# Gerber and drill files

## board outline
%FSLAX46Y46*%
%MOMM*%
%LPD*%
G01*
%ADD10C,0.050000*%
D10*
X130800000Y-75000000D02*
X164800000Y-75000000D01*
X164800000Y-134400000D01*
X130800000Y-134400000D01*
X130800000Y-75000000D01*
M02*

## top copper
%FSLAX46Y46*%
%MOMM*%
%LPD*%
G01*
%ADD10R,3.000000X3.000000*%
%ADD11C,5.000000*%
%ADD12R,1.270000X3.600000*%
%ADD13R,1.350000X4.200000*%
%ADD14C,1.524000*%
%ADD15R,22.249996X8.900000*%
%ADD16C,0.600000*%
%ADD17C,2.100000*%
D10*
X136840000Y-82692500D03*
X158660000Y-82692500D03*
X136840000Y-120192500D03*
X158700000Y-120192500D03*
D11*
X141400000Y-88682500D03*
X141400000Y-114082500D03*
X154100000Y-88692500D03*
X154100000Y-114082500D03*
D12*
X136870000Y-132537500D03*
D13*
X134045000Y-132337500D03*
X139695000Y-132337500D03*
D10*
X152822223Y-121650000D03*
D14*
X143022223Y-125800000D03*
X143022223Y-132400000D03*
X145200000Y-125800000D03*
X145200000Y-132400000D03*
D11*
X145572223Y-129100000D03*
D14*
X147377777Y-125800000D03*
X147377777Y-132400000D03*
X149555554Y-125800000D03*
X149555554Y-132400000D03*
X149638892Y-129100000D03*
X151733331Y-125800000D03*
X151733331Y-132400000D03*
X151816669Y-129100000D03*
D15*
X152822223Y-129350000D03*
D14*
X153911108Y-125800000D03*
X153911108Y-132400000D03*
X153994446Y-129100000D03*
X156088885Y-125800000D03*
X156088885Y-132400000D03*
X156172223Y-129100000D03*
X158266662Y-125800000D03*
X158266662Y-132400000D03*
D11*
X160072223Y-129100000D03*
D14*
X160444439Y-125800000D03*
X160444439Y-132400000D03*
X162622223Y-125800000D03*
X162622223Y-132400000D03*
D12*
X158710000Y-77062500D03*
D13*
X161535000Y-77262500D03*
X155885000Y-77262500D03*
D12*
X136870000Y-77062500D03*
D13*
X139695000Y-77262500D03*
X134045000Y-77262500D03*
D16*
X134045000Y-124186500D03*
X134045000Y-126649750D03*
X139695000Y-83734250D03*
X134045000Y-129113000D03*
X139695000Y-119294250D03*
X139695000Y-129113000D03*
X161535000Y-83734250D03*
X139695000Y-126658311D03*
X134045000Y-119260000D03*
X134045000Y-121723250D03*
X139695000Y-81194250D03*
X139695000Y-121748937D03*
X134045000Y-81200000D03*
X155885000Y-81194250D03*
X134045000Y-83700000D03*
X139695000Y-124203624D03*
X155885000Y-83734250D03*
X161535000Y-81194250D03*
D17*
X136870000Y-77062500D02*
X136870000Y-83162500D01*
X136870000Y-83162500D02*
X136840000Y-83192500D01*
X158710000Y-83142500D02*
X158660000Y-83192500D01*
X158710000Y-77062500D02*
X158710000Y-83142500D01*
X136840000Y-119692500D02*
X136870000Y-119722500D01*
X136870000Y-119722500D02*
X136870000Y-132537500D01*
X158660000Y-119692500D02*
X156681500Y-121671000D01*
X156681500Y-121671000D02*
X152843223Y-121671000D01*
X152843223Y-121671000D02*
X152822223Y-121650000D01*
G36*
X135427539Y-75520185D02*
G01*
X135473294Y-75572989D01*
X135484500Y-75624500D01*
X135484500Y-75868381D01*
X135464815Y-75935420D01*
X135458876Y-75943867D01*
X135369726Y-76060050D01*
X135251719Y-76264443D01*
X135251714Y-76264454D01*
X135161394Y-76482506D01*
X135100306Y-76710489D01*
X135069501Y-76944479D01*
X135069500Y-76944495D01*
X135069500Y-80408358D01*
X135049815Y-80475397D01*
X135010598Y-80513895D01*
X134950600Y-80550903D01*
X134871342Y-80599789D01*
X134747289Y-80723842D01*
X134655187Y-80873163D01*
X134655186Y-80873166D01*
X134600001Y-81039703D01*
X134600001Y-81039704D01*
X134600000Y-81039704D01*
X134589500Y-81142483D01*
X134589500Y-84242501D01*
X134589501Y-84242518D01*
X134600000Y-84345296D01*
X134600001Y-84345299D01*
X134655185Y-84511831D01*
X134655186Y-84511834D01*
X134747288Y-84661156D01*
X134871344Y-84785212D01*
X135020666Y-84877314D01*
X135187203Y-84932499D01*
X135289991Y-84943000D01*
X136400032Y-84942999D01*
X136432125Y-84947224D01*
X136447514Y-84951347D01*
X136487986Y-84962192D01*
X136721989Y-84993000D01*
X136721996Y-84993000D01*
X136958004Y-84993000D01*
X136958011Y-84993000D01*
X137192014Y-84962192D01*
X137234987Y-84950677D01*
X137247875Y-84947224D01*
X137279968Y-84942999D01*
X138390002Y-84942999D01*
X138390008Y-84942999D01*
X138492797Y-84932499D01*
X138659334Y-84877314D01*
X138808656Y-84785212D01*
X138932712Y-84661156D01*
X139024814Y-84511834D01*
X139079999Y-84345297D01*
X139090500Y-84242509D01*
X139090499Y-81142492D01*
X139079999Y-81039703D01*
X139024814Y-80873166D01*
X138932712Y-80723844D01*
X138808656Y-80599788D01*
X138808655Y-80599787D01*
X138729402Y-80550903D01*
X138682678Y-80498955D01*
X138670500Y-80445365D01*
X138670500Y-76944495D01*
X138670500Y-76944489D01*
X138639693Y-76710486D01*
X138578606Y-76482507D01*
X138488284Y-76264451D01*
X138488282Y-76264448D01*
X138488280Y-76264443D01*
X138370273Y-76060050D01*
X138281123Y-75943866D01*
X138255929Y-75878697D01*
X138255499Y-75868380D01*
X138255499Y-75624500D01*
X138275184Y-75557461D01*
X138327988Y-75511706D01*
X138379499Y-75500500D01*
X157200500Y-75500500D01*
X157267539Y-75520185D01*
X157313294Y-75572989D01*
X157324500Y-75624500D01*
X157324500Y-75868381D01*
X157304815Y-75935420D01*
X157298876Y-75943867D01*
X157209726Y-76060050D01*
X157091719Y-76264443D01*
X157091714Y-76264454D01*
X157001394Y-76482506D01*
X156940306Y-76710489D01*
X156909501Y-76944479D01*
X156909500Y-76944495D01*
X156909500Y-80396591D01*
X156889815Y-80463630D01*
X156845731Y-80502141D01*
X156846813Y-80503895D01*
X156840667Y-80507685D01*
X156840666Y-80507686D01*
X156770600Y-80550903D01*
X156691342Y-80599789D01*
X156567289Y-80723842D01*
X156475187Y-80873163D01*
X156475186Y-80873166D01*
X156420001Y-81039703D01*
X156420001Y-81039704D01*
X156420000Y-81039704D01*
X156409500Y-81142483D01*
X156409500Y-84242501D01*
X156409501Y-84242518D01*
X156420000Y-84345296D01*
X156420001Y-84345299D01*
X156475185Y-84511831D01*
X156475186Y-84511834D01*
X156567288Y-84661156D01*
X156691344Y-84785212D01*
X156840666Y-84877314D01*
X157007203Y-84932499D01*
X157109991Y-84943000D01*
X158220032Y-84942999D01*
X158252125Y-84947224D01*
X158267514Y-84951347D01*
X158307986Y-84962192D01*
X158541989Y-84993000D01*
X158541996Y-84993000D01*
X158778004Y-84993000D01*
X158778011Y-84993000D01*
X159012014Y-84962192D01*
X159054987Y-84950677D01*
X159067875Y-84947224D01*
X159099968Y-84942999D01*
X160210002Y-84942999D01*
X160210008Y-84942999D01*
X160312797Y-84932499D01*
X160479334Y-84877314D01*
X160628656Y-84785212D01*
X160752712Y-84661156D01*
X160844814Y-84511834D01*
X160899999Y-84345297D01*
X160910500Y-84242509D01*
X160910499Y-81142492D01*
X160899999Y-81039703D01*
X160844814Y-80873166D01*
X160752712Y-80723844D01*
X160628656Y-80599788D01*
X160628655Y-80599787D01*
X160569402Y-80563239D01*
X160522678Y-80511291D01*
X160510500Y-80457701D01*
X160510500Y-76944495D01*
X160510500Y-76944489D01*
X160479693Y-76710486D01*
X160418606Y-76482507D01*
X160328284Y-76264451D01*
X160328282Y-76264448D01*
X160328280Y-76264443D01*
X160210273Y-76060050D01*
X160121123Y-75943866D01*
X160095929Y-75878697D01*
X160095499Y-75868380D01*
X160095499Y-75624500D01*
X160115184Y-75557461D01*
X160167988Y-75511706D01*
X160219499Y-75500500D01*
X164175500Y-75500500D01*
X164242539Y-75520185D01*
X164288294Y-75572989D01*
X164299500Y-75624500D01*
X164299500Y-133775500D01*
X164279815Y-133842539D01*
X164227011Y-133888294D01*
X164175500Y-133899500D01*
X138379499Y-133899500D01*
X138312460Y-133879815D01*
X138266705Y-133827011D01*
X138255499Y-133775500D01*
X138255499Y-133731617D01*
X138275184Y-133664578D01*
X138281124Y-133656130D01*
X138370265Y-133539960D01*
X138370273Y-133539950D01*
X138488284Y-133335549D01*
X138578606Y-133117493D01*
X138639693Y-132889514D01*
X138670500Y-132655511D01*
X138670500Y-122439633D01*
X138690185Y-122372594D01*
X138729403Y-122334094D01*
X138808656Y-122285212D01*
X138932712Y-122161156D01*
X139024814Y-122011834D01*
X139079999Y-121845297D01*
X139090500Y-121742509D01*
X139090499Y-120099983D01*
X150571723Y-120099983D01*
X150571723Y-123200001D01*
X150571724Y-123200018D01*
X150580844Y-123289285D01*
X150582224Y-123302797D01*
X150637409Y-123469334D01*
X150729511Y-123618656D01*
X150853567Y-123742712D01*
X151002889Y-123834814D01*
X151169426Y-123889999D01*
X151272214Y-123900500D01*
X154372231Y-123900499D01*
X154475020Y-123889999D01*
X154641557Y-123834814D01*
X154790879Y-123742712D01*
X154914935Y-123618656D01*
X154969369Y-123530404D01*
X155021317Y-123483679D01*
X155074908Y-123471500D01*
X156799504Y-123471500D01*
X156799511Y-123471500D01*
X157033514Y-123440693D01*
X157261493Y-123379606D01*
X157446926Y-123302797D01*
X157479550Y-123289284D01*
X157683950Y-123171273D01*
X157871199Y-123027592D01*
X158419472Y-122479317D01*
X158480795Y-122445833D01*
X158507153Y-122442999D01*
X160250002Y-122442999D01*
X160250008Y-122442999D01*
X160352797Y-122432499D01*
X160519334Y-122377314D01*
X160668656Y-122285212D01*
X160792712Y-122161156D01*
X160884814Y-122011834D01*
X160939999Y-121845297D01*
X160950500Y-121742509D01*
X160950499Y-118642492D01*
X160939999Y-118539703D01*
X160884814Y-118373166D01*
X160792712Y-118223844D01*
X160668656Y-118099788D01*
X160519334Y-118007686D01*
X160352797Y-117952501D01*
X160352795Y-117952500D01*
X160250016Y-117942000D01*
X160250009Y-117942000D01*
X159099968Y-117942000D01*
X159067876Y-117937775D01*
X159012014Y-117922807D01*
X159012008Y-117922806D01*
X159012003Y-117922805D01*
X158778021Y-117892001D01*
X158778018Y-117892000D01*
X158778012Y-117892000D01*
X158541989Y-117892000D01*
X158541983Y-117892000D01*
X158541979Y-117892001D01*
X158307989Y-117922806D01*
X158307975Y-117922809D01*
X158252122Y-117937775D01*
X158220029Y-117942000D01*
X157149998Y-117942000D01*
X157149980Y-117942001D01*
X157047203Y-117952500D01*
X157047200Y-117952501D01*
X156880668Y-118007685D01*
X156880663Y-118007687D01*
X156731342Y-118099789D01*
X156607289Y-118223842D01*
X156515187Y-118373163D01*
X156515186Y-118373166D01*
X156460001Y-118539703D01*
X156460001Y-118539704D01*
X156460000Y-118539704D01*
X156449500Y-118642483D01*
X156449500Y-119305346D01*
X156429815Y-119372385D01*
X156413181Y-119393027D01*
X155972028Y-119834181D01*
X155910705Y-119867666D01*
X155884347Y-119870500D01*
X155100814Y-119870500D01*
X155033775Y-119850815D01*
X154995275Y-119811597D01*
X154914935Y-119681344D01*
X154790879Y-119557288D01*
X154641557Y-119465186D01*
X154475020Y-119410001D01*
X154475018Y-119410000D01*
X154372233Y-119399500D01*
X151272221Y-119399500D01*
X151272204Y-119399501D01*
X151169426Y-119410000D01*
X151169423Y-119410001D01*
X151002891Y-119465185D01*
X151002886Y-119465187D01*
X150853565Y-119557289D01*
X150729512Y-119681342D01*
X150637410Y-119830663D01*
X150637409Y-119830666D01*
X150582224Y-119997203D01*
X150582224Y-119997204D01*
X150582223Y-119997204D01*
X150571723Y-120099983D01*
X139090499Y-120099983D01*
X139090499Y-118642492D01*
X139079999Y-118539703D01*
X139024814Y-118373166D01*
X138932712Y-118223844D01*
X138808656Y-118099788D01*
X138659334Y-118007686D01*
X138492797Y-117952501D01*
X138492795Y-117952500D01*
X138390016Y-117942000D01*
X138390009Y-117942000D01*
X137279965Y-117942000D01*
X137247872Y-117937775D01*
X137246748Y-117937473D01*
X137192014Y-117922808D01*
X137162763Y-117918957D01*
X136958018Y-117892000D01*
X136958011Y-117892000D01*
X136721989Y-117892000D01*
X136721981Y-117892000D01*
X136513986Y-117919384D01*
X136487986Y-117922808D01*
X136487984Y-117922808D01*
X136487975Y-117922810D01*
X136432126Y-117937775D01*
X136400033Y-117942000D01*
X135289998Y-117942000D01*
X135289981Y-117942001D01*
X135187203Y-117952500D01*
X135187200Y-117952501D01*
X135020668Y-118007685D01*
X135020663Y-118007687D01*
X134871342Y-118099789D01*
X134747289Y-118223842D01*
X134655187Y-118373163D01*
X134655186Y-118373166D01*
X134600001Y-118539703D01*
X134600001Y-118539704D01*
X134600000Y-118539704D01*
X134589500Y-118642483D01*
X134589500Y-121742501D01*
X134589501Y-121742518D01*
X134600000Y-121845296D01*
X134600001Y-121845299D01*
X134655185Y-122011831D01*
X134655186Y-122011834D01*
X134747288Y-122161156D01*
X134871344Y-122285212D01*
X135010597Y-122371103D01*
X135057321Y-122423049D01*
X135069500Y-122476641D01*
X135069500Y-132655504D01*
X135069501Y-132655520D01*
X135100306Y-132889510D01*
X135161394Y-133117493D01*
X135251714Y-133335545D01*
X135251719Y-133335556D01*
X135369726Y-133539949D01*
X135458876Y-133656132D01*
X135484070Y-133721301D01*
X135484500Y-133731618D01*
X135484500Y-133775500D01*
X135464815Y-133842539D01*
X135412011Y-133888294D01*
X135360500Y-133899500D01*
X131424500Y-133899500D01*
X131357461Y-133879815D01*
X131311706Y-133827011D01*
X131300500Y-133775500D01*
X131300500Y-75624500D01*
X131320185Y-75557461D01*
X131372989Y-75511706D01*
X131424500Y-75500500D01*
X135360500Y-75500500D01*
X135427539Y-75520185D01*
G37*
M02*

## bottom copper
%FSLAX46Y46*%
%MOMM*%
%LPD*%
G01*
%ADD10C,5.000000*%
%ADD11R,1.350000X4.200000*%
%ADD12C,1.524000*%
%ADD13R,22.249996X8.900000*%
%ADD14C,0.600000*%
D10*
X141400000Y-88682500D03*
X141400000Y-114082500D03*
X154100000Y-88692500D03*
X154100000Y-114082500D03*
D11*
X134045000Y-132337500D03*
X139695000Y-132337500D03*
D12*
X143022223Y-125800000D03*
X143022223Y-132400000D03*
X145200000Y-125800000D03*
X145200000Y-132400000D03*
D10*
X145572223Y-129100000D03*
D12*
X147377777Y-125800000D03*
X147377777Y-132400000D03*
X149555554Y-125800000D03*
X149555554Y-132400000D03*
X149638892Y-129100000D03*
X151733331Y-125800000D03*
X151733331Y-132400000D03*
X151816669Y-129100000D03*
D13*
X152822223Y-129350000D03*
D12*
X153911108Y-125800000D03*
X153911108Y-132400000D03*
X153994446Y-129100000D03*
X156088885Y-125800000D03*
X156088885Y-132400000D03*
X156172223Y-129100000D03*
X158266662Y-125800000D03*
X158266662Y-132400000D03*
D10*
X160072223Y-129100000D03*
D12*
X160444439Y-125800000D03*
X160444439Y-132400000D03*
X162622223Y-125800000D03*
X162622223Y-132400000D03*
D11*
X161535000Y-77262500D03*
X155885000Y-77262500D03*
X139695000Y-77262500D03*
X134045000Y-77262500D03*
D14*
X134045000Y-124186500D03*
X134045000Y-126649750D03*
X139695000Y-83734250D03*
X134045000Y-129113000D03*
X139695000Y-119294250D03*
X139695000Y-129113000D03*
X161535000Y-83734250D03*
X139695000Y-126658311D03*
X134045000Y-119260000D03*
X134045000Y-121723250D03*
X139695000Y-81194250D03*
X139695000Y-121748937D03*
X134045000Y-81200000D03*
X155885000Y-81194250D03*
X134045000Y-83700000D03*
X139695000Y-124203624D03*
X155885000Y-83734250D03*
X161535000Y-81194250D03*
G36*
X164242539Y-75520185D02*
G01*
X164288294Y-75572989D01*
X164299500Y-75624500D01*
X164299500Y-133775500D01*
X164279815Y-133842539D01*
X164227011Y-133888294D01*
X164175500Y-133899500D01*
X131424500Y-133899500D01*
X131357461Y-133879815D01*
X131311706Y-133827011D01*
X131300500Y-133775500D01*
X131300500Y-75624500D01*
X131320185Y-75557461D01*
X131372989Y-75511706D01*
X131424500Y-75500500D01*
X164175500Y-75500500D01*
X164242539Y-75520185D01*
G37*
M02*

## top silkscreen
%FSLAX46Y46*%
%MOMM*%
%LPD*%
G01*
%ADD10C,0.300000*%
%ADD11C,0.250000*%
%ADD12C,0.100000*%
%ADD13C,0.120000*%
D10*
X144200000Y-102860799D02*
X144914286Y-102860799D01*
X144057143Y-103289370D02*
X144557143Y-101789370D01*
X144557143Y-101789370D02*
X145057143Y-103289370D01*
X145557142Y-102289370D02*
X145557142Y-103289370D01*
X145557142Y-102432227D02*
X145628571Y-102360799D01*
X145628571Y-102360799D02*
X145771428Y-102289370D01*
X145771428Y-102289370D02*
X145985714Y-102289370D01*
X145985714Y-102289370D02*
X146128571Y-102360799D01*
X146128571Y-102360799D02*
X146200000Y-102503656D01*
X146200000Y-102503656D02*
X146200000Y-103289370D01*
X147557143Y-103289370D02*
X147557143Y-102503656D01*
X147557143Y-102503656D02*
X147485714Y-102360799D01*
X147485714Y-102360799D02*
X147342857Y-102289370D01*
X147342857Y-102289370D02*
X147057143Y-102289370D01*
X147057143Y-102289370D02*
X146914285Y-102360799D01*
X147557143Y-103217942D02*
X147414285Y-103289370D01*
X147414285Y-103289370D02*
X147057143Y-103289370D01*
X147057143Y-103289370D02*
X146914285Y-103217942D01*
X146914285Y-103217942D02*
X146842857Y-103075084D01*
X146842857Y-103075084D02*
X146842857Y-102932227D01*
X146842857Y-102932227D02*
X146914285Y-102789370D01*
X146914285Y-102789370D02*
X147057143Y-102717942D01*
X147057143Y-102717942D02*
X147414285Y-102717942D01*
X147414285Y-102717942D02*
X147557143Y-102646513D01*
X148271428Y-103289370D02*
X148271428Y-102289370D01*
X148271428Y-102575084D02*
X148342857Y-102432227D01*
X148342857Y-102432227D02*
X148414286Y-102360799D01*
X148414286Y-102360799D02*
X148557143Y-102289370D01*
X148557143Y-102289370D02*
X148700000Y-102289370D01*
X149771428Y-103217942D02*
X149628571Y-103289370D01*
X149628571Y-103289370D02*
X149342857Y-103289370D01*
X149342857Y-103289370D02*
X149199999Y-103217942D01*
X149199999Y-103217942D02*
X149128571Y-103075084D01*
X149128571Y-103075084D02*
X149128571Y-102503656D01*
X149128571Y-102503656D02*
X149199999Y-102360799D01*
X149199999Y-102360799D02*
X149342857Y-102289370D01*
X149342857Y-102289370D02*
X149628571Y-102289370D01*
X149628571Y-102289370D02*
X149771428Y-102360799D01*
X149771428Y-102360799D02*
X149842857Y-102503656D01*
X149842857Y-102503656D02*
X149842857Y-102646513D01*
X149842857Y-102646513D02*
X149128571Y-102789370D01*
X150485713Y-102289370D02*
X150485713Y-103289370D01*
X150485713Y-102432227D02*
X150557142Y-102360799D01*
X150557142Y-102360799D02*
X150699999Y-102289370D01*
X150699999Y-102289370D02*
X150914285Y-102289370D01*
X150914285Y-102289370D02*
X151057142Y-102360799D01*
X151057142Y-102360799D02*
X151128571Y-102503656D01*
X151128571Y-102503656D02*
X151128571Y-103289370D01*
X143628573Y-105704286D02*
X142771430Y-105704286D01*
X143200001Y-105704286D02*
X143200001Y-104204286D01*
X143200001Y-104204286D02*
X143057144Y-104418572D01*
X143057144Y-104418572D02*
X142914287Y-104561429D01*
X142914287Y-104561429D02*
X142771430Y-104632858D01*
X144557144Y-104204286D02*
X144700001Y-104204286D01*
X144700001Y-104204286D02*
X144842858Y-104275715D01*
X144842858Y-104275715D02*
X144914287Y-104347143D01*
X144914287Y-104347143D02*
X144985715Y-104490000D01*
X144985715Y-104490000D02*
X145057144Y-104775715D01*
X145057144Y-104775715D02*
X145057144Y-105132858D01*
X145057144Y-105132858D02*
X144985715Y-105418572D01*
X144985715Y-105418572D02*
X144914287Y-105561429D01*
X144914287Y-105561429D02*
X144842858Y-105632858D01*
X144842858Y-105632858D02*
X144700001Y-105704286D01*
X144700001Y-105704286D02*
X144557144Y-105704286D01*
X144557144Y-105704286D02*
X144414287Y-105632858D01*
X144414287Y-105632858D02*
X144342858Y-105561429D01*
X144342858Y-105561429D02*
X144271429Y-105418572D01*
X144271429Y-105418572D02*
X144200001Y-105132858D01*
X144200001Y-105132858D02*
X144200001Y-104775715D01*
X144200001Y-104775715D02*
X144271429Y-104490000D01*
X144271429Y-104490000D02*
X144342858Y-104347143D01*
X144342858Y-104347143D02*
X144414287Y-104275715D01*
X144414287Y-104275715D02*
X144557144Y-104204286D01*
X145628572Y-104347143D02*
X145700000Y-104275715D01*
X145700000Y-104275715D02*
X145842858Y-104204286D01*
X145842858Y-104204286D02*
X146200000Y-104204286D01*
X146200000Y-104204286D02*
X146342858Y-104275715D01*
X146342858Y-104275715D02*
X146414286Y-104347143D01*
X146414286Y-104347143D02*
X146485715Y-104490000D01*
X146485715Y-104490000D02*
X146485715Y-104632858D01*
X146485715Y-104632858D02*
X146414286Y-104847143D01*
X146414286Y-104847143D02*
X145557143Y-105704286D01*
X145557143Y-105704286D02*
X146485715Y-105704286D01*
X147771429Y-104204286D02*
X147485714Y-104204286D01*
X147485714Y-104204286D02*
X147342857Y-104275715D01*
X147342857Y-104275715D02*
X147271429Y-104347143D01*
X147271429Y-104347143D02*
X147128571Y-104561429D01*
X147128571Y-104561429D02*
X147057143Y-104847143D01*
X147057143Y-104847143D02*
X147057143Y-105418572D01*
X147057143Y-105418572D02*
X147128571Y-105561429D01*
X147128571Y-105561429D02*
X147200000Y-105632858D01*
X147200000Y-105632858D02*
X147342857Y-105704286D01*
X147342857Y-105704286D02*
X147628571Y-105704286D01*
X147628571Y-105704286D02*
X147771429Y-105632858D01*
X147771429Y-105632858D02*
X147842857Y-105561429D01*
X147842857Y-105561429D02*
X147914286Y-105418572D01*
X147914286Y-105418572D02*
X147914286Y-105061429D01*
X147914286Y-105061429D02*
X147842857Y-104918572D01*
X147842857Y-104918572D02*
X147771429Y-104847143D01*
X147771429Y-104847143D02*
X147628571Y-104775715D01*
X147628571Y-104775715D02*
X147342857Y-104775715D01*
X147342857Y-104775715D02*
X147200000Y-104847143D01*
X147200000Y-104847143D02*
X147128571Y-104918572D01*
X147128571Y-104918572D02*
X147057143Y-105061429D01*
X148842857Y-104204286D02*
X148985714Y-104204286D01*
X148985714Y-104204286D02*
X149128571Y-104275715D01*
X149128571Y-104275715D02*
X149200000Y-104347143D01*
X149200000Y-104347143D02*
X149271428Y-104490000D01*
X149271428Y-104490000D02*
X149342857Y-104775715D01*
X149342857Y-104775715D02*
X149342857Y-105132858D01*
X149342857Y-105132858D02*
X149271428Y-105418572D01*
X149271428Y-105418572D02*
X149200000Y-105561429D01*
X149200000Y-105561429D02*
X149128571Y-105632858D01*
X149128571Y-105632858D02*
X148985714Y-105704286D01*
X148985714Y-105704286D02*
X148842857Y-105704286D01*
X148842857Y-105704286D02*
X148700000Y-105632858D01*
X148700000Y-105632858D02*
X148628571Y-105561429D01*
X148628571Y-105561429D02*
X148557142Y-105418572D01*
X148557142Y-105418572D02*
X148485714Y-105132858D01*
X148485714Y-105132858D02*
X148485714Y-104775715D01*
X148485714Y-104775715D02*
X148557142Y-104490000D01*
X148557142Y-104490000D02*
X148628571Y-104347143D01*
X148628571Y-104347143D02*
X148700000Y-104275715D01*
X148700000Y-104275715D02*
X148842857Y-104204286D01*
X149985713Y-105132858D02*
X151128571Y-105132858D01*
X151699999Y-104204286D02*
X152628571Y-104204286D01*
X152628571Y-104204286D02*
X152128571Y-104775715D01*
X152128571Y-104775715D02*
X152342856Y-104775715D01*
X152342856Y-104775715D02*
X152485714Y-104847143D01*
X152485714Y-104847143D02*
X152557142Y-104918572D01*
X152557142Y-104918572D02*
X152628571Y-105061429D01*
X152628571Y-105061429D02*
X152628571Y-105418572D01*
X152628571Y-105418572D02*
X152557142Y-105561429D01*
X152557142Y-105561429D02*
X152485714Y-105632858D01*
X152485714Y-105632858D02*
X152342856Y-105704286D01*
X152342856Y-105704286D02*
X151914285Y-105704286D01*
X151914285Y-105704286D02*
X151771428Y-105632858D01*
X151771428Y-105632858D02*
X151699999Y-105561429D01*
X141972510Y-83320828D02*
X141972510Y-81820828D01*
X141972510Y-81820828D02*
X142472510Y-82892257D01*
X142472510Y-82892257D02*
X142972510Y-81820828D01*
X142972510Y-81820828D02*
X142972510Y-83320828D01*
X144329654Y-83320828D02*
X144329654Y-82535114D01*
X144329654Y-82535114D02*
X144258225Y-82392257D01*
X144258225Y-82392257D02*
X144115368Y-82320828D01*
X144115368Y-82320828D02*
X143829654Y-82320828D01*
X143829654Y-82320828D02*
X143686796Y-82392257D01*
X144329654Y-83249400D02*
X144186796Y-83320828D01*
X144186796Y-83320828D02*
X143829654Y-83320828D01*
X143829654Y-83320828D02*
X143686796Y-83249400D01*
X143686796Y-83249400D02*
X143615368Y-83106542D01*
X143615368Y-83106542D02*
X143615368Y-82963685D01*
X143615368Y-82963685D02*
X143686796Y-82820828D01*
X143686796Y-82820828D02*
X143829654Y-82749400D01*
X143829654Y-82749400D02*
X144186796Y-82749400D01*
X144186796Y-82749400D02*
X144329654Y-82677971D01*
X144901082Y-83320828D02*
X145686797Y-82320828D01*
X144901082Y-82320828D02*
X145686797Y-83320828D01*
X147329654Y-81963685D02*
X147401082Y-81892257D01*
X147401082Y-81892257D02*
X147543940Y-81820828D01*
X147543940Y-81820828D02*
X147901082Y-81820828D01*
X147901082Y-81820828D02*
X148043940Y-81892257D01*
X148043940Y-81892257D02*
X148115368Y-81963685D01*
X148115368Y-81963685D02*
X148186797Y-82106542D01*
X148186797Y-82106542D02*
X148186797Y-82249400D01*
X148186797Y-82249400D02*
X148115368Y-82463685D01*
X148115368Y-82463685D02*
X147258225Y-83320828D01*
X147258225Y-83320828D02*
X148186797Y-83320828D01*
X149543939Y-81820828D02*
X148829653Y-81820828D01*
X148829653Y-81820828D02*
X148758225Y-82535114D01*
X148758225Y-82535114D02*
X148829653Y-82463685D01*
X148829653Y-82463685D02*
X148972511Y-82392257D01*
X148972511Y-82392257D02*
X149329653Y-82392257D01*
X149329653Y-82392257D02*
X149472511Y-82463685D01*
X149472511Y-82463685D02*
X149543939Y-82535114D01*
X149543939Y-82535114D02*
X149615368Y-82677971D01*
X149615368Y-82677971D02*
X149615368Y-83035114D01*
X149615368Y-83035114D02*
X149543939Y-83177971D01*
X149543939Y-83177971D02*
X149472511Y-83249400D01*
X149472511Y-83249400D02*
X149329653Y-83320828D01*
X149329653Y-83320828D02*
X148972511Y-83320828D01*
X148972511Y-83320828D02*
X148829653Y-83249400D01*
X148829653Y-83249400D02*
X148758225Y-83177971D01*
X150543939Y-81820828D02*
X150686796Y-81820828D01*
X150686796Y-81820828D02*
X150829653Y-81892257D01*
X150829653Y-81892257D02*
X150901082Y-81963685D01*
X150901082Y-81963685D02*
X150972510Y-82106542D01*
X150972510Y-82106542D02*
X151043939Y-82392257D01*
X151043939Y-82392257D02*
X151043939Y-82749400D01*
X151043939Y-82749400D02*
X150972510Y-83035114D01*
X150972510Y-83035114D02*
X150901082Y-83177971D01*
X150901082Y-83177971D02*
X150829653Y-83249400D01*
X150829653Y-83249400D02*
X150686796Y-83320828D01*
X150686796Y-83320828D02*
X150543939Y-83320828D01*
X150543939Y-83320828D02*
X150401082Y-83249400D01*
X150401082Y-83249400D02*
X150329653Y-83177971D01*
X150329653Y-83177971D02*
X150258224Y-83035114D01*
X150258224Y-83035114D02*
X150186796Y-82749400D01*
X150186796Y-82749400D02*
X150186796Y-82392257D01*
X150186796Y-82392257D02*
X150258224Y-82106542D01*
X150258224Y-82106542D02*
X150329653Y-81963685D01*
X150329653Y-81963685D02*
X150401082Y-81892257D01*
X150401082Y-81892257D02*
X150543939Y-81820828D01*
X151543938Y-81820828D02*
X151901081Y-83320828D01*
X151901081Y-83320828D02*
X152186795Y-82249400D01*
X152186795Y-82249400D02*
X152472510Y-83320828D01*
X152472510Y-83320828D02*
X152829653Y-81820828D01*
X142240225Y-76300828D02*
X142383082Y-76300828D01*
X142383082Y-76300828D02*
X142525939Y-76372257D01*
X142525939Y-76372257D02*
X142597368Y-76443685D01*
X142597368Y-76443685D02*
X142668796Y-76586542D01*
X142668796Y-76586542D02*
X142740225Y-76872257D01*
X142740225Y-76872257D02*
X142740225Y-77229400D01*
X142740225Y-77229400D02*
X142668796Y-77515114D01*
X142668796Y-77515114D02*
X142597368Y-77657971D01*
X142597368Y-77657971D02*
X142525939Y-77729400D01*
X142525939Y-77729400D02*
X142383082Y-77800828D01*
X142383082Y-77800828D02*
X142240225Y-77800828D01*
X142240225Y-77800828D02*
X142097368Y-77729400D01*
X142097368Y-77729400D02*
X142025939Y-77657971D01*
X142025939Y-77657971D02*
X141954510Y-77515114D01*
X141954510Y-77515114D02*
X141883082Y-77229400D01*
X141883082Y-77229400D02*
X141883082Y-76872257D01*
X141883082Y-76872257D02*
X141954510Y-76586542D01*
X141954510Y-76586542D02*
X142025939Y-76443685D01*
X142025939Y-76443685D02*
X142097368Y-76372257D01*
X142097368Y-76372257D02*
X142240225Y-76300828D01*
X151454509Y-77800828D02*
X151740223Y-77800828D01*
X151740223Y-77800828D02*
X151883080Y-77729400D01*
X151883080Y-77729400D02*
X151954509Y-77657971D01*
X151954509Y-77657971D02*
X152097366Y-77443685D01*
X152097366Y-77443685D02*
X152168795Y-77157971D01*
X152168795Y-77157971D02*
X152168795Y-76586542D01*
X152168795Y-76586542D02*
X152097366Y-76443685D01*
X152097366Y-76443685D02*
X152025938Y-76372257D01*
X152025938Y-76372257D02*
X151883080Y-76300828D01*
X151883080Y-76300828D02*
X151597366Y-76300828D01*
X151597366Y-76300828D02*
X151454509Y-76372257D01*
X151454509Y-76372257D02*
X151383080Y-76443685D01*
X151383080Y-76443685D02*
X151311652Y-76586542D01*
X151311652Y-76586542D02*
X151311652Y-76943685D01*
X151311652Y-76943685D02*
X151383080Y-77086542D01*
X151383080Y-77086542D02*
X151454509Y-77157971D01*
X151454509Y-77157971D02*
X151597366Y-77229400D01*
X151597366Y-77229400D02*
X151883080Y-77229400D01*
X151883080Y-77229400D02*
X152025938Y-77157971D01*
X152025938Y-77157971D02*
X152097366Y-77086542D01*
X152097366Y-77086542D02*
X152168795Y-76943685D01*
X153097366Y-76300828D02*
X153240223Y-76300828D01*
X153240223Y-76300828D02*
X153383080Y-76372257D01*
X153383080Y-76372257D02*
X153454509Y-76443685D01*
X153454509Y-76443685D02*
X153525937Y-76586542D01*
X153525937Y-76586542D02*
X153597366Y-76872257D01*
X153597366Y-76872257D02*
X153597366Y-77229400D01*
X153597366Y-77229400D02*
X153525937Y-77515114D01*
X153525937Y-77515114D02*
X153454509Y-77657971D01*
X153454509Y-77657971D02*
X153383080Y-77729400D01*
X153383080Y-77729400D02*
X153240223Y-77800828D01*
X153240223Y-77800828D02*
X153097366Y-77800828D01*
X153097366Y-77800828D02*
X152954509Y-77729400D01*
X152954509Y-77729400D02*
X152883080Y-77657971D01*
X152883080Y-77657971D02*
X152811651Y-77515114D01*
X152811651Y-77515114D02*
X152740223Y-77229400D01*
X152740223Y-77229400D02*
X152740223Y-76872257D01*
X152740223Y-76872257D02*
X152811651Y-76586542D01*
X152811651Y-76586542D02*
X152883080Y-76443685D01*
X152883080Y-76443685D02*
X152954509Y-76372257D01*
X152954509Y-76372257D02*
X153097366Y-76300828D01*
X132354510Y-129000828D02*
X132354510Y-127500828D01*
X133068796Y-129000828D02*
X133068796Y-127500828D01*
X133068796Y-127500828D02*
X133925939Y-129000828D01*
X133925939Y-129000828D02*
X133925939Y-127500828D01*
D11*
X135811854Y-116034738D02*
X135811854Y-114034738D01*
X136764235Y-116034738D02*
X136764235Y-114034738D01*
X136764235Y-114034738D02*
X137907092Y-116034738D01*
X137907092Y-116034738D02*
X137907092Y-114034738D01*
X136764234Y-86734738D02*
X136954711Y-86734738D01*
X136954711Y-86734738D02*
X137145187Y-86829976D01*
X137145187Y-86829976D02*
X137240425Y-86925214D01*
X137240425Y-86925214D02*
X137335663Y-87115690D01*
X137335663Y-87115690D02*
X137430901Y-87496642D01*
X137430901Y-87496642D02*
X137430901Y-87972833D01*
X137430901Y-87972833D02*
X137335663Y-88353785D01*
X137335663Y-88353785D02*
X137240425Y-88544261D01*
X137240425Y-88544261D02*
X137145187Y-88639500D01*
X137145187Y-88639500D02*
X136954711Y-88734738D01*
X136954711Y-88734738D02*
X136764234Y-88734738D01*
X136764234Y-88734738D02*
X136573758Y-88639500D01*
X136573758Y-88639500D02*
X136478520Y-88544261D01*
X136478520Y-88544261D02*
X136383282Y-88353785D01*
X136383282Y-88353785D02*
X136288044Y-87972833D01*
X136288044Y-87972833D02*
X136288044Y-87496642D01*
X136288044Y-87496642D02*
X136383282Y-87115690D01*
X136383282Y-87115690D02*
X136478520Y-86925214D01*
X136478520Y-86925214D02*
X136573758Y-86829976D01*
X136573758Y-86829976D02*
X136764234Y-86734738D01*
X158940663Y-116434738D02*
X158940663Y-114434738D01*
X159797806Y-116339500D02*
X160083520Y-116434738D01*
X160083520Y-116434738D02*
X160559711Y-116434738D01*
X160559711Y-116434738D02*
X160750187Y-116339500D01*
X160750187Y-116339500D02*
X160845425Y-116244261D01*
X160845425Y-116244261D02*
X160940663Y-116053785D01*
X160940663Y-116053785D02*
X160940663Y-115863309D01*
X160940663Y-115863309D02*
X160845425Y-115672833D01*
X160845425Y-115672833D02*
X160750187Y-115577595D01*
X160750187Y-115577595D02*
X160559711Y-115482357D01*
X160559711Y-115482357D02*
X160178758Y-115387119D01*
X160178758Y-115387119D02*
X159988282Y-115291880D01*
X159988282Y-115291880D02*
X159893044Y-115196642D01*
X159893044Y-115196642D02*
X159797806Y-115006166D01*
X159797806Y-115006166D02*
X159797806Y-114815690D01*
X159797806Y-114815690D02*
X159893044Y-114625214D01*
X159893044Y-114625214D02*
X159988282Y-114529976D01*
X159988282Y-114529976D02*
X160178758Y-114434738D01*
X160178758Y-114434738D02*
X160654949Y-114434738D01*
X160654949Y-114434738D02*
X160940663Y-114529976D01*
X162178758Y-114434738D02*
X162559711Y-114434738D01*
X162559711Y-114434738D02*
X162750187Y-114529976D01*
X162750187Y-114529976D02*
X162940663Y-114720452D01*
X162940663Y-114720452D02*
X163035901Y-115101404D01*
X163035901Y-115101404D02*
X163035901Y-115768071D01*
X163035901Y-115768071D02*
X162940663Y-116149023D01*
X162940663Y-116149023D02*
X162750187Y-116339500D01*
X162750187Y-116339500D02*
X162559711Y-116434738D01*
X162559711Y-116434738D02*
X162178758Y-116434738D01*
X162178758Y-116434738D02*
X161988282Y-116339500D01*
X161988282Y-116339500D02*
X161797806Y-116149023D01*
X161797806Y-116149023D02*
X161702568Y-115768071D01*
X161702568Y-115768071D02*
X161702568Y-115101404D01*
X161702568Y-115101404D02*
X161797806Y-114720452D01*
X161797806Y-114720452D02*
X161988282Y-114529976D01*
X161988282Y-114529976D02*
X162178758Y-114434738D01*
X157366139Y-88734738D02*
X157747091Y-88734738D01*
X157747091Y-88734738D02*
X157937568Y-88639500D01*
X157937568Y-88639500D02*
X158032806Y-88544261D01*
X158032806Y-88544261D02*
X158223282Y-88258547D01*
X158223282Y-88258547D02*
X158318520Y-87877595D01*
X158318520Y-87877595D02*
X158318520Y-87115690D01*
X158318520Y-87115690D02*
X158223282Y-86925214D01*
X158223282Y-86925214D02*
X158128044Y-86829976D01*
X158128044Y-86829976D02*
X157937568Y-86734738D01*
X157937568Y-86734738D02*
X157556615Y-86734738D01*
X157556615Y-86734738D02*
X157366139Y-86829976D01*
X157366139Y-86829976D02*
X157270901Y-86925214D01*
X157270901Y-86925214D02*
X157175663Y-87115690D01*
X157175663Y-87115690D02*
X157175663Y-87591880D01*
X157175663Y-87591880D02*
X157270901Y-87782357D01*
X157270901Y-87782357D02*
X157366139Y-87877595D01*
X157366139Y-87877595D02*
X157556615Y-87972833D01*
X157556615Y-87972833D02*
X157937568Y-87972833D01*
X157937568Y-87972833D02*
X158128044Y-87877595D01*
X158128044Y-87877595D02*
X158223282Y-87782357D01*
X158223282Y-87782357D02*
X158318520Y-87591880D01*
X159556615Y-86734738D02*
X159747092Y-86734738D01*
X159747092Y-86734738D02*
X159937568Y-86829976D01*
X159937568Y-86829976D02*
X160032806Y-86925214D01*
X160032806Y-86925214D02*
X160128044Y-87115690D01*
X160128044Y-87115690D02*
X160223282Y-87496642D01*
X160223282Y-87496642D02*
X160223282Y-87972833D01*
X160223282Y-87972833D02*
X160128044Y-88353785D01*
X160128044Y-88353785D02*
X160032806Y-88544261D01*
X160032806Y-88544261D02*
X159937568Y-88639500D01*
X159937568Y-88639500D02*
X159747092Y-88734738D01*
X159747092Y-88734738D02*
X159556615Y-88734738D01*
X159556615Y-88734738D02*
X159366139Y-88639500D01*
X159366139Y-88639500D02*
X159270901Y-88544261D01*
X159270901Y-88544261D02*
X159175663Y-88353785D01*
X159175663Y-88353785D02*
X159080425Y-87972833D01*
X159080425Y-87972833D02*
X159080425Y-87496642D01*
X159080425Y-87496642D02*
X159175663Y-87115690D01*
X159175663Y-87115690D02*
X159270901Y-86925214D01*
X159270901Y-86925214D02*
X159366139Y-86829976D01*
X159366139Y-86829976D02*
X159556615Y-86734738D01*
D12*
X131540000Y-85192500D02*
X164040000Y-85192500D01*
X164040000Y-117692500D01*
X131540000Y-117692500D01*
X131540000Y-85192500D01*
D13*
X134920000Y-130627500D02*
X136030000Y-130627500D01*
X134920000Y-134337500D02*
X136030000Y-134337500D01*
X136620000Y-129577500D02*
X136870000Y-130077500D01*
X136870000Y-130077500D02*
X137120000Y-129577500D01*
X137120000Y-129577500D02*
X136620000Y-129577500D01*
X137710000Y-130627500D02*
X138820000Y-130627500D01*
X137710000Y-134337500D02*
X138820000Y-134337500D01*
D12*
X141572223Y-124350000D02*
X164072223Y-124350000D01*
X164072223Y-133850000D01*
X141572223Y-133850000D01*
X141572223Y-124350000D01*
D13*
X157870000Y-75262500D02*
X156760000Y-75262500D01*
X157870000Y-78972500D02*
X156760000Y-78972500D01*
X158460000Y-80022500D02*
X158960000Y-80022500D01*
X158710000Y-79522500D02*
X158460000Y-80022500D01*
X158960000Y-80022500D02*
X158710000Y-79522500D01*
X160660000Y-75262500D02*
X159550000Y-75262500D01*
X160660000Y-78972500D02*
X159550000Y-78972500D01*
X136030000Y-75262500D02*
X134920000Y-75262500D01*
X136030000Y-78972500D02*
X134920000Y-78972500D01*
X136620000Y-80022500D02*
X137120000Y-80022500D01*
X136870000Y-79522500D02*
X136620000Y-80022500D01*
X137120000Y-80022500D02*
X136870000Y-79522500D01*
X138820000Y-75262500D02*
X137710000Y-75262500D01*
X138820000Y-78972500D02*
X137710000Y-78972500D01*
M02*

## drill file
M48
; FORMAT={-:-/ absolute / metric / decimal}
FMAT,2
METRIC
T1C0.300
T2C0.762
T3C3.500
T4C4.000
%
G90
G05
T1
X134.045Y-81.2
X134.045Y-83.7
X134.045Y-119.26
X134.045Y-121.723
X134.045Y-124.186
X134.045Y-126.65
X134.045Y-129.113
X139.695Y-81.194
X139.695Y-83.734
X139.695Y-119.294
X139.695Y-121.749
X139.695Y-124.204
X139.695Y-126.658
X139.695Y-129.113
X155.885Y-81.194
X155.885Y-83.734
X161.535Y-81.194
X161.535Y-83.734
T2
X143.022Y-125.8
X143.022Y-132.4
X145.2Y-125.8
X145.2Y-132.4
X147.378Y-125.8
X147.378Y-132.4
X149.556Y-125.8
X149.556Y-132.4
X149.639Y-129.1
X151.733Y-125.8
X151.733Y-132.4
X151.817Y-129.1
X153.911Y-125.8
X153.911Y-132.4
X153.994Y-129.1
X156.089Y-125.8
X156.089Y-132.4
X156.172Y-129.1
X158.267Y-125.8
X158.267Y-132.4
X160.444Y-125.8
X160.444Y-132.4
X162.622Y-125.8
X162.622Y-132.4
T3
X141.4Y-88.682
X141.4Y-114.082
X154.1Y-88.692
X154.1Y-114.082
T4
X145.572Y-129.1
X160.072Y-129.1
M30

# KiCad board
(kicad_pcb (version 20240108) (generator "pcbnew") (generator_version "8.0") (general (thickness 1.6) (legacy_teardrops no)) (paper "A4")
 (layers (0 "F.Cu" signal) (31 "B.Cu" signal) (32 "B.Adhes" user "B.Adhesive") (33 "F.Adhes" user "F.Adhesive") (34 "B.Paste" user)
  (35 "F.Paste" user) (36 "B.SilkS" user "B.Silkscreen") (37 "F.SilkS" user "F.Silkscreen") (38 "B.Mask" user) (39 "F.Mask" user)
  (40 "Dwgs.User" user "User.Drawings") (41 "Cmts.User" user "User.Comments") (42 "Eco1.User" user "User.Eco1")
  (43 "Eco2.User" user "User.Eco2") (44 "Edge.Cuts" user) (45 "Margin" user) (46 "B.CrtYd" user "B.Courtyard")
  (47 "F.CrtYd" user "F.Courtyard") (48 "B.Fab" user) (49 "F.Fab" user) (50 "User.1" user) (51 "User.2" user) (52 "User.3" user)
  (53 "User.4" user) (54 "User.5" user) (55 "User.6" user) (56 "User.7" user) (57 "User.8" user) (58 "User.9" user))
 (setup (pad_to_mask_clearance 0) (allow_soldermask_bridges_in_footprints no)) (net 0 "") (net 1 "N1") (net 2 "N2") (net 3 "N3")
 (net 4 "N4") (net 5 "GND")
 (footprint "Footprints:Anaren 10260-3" (layer "F.Cu") (at 148.7 101.6925)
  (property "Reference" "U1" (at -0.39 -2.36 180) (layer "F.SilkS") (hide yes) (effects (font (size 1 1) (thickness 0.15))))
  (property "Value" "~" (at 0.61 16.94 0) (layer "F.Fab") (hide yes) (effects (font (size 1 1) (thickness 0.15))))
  (fp_rect (start -17.16 -16.5) (end 15.34 16) (stroke (width 0.1) (type default)) (fill none) (layer "F.SilkS"))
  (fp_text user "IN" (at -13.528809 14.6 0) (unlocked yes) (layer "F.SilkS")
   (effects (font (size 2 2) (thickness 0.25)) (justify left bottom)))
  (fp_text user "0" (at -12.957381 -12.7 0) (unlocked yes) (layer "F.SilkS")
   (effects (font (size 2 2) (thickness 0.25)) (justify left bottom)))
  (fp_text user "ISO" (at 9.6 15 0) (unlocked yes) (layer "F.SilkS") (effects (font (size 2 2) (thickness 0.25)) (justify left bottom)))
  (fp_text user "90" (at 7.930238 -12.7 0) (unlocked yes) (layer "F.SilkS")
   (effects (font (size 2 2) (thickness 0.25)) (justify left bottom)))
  (pad "1" smd rect (at -11.86 -19 270) (size 3 3) (layers "F.Cu" "F.Paste" "F.Mask") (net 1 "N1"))
  (pad "2" smd rect (at 9.96 -19 270) (size 3 3) (layers "F.Cu" "F.Paste" "F.Mask") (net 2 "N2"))
  (pad "3" smd rect (at -11.86 18.5 270) (size 3 3) (layers "F.Cu" "F.Paste" "F.Mask") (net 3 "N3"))
  (pad "4" smd rect (at 10 18.5 270) (size 3 3) (layers "F.Cu" "F.Paste" "F.Mask") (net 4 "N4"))
  (pad "5" thru_hole circle (at -7.3 -13.01) (size 5 5) (drill 3.5) (layers "*.Cu" "*.Mask") (remove_unused_layers no) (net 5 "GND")
   (zone_connect 2))
  (pad "5" thru_hole circle (at -7.3 12.39) (size 5 5) (drill 3.5) (layers "*.Cu" "*.Mask") (remove_unused_layers no) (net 5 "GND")
   (zone_connect 2))
  (pad "5" thru_hole circle (at 5.4 -13) (size 5 5) (drill 3.5) (layers "*.Cu" "*.Mask") (remove_unused_layers no) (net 5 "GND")
   (zone_connect 2))
  (pad "5" thru_hole circle (at 5.4 12.39) (size 5 5) (drill 3.5) (layers "*.Cu" "*.Mask") (remove_unused_layers no) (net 5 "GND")
   (zone_connect 2)))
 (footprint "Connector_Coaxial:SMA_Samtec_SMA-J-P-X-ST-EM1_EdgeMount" (layer "F.Cu") (at 136.87 132.3375)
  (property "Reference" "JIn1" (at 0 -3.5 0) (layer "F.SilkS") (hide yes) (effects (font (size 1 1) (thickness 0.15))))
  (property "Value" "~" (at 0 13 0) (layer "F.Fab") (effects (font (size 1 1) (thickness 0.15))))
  (fp_line (start -1.95 -1.71) (end -0.84 -1.71) (stroke (width 0.12) (type solid)) (layer "F.SilkS"))
  (fp_line (start -1.95 2) (end -0.84 2) (stroke (width 0.12) (type solid)) (layer "F.SilkS"))
  (fp_line (start -0.25 -2.76) (end 0 -2.26) (stroke (width 0.12) (type solid)) (layer "F.SilkS"))
  (fp_line (start 0 -2.26) (end 0.25 -2.76) (stroke (width 0.12) (type solid)) (layer "F.SilkS"))
  (fp_line (start 0.25 -2.76) (end -0.25 -2.76) (stroke (width 0.12) (type solid)) (layer "F.SilkS"))
  (fp_line (start 0.84 -1.71) (end 1.95 -1.71) (stroke (width 0.12) (type solid)) (layer "F.SilkS"))
  (fp_line (start 0.84 2) (end 1.95 2) (stroke (width 0.12) (type solid)) (layer "F.SilkS"))
  (pad "1" smd rect (at 0 0.2) (size 1.27 3.6) (layers "F.Cu" "F.Paste" "F.Mask") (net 3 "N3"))
  (pad "2" smd rect (at -2.825 0) (size 1.35 4.2) (layers "F.Cu" "F.Paste" "F.Mask") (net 5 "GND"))
  (pad "2" smd rect (at -2.825 0) (size 1.35 4.2) (layers "B.Cu" "B.Paste" "B.Mask") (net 5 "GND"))
  (pad "2" smd rect (at 2.825 0) (size 1.35 4.2) (layers "F.Cu" "F.Paste" "F.Mask") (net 5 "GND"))
  (pad "2" smd rect (at 2.825 0) (size 1.35 4.2) (layers "B.Cu" "B.Paste" "B.Mask") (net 5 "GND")))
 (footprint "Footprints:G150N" (layer "F.Cu") (at 152.822223 129.65)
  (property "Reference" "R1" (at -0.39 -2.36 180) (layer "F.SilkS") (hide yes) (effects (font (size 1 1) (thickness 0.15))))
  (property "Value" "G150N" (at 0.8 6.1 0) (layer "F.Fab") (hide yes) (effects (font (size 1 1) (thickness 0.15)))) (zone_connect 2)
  (fp_rect (start -11.25 -5.3) (end 11.25 4.2) (stroke (width 0.1) (type default)) (fill none) (layer "F.SilkS"))
  (pad "1" smd rect (at 0 -8 270) (size 3 3) (layers "F.Cu" "F.Paste" "F.Mask") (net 4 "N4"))
  (pad "2" thru_hole circle (at -9.8 -3.85) (size 1.524 1.524) (drill 0.762) (layers "*.Cu" "*.Mask") (remove_unused_layers no)
   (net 5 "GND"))
  (pad "2" thru_hole circle (at -9.8 2.75) (size 1.524 1.524) (drill 0.762) (layers "*.Cu" "*.Mask") (remove_unused_layers no) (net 5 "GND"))
  (pad "2" thru_hole circle (at -7.622223 -3.85) (size 1.524 1.524) (drill 0.762) (layers "*.Cu" "*.Mask") (remove_unused_layers no)
   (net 5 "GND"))
  (pad "2" thru_hole circle (at -7.622223 2.75) (size 1.524 1.524) (drill 0.762) (layers "*.Cu" "*.Mask") (remove_unused_layers no)
   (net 5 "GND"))
  (pad "2" thru_hole circle (at -7.25 -0.55 270) (size 5 5) (drill 4) (layers "*.Cu" "*.Mask") (remove_unused_layers no) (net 5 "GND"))
  (pad "2" thru_hole circle (at -5.444446 -3.85) (size 1.524 1.524) (drill 0.762) (layers "*.Cu" "*.Mask") (remove_unused_layers no)
   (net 5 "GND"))
  (pad "2" thru_hole circle (at -5.444446 2.75) (size 1.524 1.524) (drill 0.762) (layers "*.Cu" "*.Mask") (remove_unused_layers no)
   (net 5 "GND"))
  (pad "2" thru_hole circle (at -3.266669 -3.85) (size 1.524 1.524) (drill 0.762) (layers "*.Cu" "*.Mask") (remove_unused_layers no)
   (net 5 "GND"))
  (pad "2" thru_hole circle (at -3.266669 2.75) (size 1.524 1.524) (drill 0.762) (layers "*.Cu" "*.Mask") (remove_unused_layers no)
   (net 5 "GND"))
  (pad "2" thru_hole circle (at -3.183331 -0.55) (size 1.524 1.524) (drill 0.762) (layers "*.Cu" "*.Mask") (remove_unused_layers no)
   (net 5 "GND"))
  (pad "2" thru_hole circle (at -1.088892 -3.85) (size 1.524 1.524) (drill 0.762) (layers "*.Cu" "*.Mask") (remove_unused_layers no)
   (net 5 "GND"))
  (pad "2" thru_hole circle (at -1.088892 2.75) (size 1.524 1.524) (drill 0.762) (layers "*.Cu" "*.Mask") (remove_unused_layers no)
   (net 5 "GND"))
  (pad "2" thru_hole circle (at -1.005554 -0.55) (size 1.524 1.524) (drill 0.762) (layers "*.Cu" "*.Mask") (remove_unused_layers no)
   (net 5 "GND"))
  (pad "2" smd rect (at 0 -0.3 270) (size 8.9 22.249996) (layers "F.Cu" "F.Mask") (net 5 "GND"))
  (pad "2" smd rect (at 0 -0.3 270) (size 8.9 22.249996) (layers "B.Cu" "B.Mask") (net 5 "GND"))
  (pad "2" thru_hole circle (at 1.088885 -3.85) (size 1.524 1.524) (drill 0.762) (layers "*.Cu" "*.Mask") (remove_unused_layers no)
   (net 5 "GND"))
  (pad "2" thru_hole circle (at 1.088885 2.75) (size 1.524 1.524) (drill 0.762) (layers "*.Cu" "*.Mask") (remove_unused_layers no)
   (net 5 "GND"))
  (pad "2" thru_hole circle (at 1.172223 -0.55) (size 1.524 1.524) (drill 0.762) (layers "*.Cu" "*.Mask") (remove_unused_layers no)
   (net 5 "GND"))
  (pad "2" thru_hole circle (at 3.266662 -3.85) (size 1.524 1.524) (drill 0.762) (layers "*.Cu" "*.Mask") (remove_unused_layers no)
   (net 5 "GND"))
  (pad "2" thru_hole circle (at 3.266662 2.75) (size 1.524 1.524) (drill 0.762) (layers "*.Cu" "*.Mask") (remove_unused_layers no)
   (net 5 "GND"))
  (pad "2" thru_hole circle (at 3.35 -0.55) (size 1.524 1.524) (drill 0.762) (layers "*.Cu" "*.Mask") (remove_unused_layers no)
   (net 5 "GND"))
  (pad "2" thru_hole circle (at 5.444439 -3.85) (size 1.524 1.524) (drill 0.762) (layers "*.Cu" "*.Mask") (remove_unused_layers no)
   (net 5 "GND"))
  (pad "2" thru_hole circle (at 5.444439 2.75) (size 1.524 1.524) (drill 0.762) (layers "*.Cu" "*.Mask") (remove_unused_layers no)
   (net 5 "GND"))
  (pad "2" thru_hole circle (at 7.25 -0.55 270) (size 5 5) (drill 4) (layers "*.Cu" "*.Mask") (remove_unused_layers no) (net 5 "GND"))
  (pad "2" thru_hole circle (at 7.622216 -3.85) (size 1.524 1.524) (drill 0.762) (layers "*.Cu" "*.Mask") (remove_unused_layers no)
   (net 5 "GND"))
  (pad "2" thru_hole circle (at 7.622216 2.75) (size 1.524 1.524) (drill 0.762) (layers "*.Cu" "*.Mask") (remove_unused_layers no)
   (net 5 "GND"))
  (pad "2" thru_hole circle (at 9.8 -3.85) (size 1.524 1.524) (drill 0.762) (layers "*.Cu" "*.Mask") (remove_unused_layers no) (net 5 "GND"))
  (pad "2" thru_hole circle (at 9.8 2.75) (size 1.524 1.524) (drill 0.762) (layers "*.Cu" "*.Mask") (remove_unused_layers no) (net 5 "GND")))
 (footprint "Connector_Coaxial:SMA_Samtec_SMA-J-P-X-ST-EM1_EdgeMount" (layer "F.Cu") (at 158.71 77.2625 180)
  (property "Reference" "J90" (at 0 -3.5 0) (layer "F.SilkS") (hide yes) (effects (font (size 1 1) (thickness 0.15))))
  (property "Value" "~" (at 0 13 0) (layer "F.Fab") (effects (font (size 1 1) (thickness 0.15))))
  (fp_line (start 0.84 2) (end 1.95 2) (stroke (width 0.12) (type solid)) (layer "F.SilkS"))
  (fp_line (start 0.84 -1.71) (end 1.95 -1.71) (stroke (width 0.12) (type solid)) (layer "F.SilkS"))
  (fp_line (start 0.25 -2.76) (end -0.25 -2.76) (stroke (width 0.12) (type solid)) (layer "F.SilkS"))
  (fp_line (start 0 -2.26) (end 0.25 -2.76) (stroke (width 0.12) (type solid)) (layer "F.SilkS"))
  (fp_line (start -0.25 -2.76) (end 0 -2.26) (stroke (width 0.12) (type solid)) (layer "F.SilkS"))
  (fp_line (start -1.95 2) (end -0.84 2) (stroke (width 0.12) (type solid)) (layer "F.SilkS"))
  (fp_line (start -1.95 -1.71) (end -0.84 -1.71) (stroke (width 0.12) (type solid)) (layer "F.SilkS"))
  (pad "1" smd rect (at 0 0.2 180) (size 1.27 3.6) (layers "F.Cu" "F.Paste" "F.Mask") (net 2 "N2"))
  (pad "2" smd rect (at -2.825 0 180) (size 1.35 4.2) (layers "F.Cu" "F.Paste" "F.Mask") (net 5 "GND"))
  (pad "2" smd rect (at -2.825 0 180) (size 1.35 4.2) (layers "B.Cu" "B.Paste" "B.Mask") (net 5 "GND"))
  (pad "2" smd rect (at 2.825 0 180) (size 1.35 4.2) (layers "F.Cu" "F.Paste" "F.Mask") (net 5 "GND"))
  (pad "2" smd rect (at 2.825 0 180) (size 1.35 4.2) (layers "B.Cu" "B.Paste" "B.Mask") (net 5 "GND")))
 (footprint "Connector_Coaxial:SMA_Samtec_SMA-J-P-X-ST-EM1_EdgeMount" (layer "F.Cu") (at 136.87 77.2625 180)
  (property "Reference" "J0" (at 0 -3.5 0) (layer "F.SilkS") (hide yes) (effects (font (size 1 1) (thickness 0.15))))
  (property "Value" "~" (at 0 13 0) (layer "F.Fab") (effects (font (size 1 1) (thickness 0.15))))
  (fp_line (start 0.84 2) (end 1.95 2) (stroke (width 0.12) (type solid)) (layer "F.SilkS"))
  (fp_line (start 0.84 -1.71) (end 1.95 -1.71) (stroke (width 0.12) (type solid)) (layer "F.SilkS"))
  (fp_line (start 0.25 -2.76) (end -0.25 -2.76) (stroke (width 0.12) (type solid)) (layer "F.SilkS"))
  (fp_line (start 0 -2.26) (end 0.25 -2.76) (stroke (width 0.12) (type solid)) (layer "F.SilkS"))
  (fp_line (start -0.25 -2.76) (end 0 -2.26) (stroke (width 0.12) (type solid)) (layer "F.SilkS"))
  (fp_line (start -1.95 2) (end -0.84 2) (stroke (width 0.12) (type solid)) (layer "F.SilkS"))
  (fp_line (start -1.95 -1.71) (end -0.84 -1.71) (stroke (width 0.12) (type solid)) (layer "F.SilkS"))
  (pad "1" smd rect (at 0 0.2 180) (size 1.27 3.6) (layers "F.Cu" "F.Paste" "F.Mask") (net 1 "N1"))
  (pad "2" smd rect (at -2.825 0 180) (size 1.35 4.2) (layers "F.Cu" "F.Paste" "F.Mask") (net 5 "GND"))
  (pad "2" smd rect (at -2.825 0 180) (size 1.35 4.2) (layers "B.Cu" "B.Paste" "B.Mask") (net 5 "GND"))
  (pad "2" smd rect (at 2.825 0 180) (size 1.35 4.2) (layers "F.Cu" "F.Paste" "F.Mask") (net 5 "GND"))
  (pad "2" smd rect (at 2.825 0 180) (size 1.35 4.2) (layers "B.Cu" "B.Paste" "B.Mask") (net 5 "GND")))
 (gr_rect (start 130.8 75) (end 164.8 134.4) (stroke (width 0.05) (type default)) (fill none) (layer "Edge.Cuts"))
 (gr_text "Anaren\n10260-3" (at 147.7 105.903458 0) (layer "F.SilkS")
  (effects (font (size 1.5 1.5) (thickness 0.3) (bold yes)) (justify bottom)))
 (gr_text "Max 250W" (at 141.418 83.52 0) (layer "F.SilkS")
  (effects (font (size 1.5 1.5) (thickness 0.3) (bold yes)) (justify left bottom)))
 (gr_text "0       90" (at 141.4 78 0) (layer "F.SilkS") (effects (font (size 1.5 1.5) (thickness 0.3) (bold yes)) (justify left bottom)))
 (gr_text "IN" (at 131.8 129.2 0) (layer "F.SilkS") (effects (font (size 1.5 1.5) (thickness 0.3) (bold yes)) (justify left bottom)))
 (via (at 134.045 124.1865) (size 0.6) (drill 0.3) (layers "F.Cu" "B.Cu") (free yes) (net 5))
 (via (at 134.045 126.64975) (size 0.6) (drill 0.3) (layers "F.Cu" "B.Cu") (free yes) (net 5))
 (via (at 139.695 83.73425) (size 0.6) (drill 0.3) (layers "F.Cu" "B.Cu") (free yes) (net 5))
 (via (at 134.045 129.113) (size 0.6) (drill 0.3) (layers "F.Cu" "B.Cu") (free yes) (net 5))
 (via (at 139.695 119.29425) (size 0.6) (drill 0.3) (layers "F.Cu" "B.Cu") (free yes) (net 5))
 (via (at 139.695 129.113) (size 0.6) (drill 0.3) (layers "F.Cu" "B.Cu") (free yes) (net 5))
 (via (at 161.535 83.73425) (size 0.6) (drill 0.3) (layers "F.Cu" "B.Cu") (free yes) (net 5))
 (via (at 139.695 126.658311) (size 0.6) (drill 0.3) (layers "F.Cu" "B.Cu") (free yes) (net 5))
 (via (at 134.045 119.26) (size 0.6) (drill 0.3) (layers "F.Cu" "B.Cu") (free yes) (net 5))
 (via (at 134.045 121.72325) (size 0.6) (drill 0.3) (layers "F.Cu" "B.Cu") (free yes) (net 5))
 (via (at 139.695 81.19425) (size 0.6) (drill 0.3) (layers "F.Cu" "B.Cu") (free yes) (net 5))
 (via (at 139.695 121.748937) (size 0.6) (drill 0.3) (layers "F.Cu" "B.Cu") (free yes) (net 5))
 (via (at 134.045 81.2) (size 0.6) (drill 0.3) (layers "F.Cu" "B.Cu") (free yes) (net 5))
 (via (at 155.885 81.19425) (size 0.6) (drill 0.3) (layers "F.Cu" "B.Cu") (free yes) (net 5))
 (via (at 134.045 83.7) (size 0.6) (drill 0.3) (layers "F.Cu" "B.Cu") (free yes) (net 5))
 (via (at 139.695 124.203624) (size 0.6) (drill 0.3) (layers "F.Cu" "B.Cu") (free yes) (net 5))
 (via (at 155.885 83.73425) (size 0.6) (drill 0.3) (layers "F.Cu" "B.Cu") (free yes) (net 5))
 (via (at 161.535 81.19425) (size 0.6) (drill 0.3) (layers "F.Cu" "B.Cu") (free yes) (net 5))
 (segment (start 136.87 77.0625) (end 136.87 83.1625) (width 2.1) (layer "F.Cu") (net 1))
 (segment (start 136.87 83.1625) (end 136.84 83.1925) (width 2.1) (layer "F.Cu") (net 1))
 (segment (start 158.71 83.1425) (end 158.66 83.1925) (width 2.1) (layer "F.Cu") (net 2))
 (segment (start 158.71 77.0625) (end 158.71 83.1425) (width 2.1) (layer "F.Cu") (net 2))
 (segment (start 136.84 119.6925) (end 136.87 119.7225) (width 2.1) (layer "F.Cu") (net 3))
 (segment (start 136.87 119.7225) (end 136.87 132.5375) (width 2.1) (layer "F.Cu") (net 3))
 (segment (start 158.66 119.6925) (end 156.6815 121.671) (width 2.1) (layer "F.Cu") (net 4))
 (segment (start 156.6815 121.671) (end 152.843223 121.671) (width 2.1) (layer "F.Cu") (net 4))
 (segment (start 152.843223 121.671) (end 152.822223 121.65) (width 2.1) (layer "F.Cu") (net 4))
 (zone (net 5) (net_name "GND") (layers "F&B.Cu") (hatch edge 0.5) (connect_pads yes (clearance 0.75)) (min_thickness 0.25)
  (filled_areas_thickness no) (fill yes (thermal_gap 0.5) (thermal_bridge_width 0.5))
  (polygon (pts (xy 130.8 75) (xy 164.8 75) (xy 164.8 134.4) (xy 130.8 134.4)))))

